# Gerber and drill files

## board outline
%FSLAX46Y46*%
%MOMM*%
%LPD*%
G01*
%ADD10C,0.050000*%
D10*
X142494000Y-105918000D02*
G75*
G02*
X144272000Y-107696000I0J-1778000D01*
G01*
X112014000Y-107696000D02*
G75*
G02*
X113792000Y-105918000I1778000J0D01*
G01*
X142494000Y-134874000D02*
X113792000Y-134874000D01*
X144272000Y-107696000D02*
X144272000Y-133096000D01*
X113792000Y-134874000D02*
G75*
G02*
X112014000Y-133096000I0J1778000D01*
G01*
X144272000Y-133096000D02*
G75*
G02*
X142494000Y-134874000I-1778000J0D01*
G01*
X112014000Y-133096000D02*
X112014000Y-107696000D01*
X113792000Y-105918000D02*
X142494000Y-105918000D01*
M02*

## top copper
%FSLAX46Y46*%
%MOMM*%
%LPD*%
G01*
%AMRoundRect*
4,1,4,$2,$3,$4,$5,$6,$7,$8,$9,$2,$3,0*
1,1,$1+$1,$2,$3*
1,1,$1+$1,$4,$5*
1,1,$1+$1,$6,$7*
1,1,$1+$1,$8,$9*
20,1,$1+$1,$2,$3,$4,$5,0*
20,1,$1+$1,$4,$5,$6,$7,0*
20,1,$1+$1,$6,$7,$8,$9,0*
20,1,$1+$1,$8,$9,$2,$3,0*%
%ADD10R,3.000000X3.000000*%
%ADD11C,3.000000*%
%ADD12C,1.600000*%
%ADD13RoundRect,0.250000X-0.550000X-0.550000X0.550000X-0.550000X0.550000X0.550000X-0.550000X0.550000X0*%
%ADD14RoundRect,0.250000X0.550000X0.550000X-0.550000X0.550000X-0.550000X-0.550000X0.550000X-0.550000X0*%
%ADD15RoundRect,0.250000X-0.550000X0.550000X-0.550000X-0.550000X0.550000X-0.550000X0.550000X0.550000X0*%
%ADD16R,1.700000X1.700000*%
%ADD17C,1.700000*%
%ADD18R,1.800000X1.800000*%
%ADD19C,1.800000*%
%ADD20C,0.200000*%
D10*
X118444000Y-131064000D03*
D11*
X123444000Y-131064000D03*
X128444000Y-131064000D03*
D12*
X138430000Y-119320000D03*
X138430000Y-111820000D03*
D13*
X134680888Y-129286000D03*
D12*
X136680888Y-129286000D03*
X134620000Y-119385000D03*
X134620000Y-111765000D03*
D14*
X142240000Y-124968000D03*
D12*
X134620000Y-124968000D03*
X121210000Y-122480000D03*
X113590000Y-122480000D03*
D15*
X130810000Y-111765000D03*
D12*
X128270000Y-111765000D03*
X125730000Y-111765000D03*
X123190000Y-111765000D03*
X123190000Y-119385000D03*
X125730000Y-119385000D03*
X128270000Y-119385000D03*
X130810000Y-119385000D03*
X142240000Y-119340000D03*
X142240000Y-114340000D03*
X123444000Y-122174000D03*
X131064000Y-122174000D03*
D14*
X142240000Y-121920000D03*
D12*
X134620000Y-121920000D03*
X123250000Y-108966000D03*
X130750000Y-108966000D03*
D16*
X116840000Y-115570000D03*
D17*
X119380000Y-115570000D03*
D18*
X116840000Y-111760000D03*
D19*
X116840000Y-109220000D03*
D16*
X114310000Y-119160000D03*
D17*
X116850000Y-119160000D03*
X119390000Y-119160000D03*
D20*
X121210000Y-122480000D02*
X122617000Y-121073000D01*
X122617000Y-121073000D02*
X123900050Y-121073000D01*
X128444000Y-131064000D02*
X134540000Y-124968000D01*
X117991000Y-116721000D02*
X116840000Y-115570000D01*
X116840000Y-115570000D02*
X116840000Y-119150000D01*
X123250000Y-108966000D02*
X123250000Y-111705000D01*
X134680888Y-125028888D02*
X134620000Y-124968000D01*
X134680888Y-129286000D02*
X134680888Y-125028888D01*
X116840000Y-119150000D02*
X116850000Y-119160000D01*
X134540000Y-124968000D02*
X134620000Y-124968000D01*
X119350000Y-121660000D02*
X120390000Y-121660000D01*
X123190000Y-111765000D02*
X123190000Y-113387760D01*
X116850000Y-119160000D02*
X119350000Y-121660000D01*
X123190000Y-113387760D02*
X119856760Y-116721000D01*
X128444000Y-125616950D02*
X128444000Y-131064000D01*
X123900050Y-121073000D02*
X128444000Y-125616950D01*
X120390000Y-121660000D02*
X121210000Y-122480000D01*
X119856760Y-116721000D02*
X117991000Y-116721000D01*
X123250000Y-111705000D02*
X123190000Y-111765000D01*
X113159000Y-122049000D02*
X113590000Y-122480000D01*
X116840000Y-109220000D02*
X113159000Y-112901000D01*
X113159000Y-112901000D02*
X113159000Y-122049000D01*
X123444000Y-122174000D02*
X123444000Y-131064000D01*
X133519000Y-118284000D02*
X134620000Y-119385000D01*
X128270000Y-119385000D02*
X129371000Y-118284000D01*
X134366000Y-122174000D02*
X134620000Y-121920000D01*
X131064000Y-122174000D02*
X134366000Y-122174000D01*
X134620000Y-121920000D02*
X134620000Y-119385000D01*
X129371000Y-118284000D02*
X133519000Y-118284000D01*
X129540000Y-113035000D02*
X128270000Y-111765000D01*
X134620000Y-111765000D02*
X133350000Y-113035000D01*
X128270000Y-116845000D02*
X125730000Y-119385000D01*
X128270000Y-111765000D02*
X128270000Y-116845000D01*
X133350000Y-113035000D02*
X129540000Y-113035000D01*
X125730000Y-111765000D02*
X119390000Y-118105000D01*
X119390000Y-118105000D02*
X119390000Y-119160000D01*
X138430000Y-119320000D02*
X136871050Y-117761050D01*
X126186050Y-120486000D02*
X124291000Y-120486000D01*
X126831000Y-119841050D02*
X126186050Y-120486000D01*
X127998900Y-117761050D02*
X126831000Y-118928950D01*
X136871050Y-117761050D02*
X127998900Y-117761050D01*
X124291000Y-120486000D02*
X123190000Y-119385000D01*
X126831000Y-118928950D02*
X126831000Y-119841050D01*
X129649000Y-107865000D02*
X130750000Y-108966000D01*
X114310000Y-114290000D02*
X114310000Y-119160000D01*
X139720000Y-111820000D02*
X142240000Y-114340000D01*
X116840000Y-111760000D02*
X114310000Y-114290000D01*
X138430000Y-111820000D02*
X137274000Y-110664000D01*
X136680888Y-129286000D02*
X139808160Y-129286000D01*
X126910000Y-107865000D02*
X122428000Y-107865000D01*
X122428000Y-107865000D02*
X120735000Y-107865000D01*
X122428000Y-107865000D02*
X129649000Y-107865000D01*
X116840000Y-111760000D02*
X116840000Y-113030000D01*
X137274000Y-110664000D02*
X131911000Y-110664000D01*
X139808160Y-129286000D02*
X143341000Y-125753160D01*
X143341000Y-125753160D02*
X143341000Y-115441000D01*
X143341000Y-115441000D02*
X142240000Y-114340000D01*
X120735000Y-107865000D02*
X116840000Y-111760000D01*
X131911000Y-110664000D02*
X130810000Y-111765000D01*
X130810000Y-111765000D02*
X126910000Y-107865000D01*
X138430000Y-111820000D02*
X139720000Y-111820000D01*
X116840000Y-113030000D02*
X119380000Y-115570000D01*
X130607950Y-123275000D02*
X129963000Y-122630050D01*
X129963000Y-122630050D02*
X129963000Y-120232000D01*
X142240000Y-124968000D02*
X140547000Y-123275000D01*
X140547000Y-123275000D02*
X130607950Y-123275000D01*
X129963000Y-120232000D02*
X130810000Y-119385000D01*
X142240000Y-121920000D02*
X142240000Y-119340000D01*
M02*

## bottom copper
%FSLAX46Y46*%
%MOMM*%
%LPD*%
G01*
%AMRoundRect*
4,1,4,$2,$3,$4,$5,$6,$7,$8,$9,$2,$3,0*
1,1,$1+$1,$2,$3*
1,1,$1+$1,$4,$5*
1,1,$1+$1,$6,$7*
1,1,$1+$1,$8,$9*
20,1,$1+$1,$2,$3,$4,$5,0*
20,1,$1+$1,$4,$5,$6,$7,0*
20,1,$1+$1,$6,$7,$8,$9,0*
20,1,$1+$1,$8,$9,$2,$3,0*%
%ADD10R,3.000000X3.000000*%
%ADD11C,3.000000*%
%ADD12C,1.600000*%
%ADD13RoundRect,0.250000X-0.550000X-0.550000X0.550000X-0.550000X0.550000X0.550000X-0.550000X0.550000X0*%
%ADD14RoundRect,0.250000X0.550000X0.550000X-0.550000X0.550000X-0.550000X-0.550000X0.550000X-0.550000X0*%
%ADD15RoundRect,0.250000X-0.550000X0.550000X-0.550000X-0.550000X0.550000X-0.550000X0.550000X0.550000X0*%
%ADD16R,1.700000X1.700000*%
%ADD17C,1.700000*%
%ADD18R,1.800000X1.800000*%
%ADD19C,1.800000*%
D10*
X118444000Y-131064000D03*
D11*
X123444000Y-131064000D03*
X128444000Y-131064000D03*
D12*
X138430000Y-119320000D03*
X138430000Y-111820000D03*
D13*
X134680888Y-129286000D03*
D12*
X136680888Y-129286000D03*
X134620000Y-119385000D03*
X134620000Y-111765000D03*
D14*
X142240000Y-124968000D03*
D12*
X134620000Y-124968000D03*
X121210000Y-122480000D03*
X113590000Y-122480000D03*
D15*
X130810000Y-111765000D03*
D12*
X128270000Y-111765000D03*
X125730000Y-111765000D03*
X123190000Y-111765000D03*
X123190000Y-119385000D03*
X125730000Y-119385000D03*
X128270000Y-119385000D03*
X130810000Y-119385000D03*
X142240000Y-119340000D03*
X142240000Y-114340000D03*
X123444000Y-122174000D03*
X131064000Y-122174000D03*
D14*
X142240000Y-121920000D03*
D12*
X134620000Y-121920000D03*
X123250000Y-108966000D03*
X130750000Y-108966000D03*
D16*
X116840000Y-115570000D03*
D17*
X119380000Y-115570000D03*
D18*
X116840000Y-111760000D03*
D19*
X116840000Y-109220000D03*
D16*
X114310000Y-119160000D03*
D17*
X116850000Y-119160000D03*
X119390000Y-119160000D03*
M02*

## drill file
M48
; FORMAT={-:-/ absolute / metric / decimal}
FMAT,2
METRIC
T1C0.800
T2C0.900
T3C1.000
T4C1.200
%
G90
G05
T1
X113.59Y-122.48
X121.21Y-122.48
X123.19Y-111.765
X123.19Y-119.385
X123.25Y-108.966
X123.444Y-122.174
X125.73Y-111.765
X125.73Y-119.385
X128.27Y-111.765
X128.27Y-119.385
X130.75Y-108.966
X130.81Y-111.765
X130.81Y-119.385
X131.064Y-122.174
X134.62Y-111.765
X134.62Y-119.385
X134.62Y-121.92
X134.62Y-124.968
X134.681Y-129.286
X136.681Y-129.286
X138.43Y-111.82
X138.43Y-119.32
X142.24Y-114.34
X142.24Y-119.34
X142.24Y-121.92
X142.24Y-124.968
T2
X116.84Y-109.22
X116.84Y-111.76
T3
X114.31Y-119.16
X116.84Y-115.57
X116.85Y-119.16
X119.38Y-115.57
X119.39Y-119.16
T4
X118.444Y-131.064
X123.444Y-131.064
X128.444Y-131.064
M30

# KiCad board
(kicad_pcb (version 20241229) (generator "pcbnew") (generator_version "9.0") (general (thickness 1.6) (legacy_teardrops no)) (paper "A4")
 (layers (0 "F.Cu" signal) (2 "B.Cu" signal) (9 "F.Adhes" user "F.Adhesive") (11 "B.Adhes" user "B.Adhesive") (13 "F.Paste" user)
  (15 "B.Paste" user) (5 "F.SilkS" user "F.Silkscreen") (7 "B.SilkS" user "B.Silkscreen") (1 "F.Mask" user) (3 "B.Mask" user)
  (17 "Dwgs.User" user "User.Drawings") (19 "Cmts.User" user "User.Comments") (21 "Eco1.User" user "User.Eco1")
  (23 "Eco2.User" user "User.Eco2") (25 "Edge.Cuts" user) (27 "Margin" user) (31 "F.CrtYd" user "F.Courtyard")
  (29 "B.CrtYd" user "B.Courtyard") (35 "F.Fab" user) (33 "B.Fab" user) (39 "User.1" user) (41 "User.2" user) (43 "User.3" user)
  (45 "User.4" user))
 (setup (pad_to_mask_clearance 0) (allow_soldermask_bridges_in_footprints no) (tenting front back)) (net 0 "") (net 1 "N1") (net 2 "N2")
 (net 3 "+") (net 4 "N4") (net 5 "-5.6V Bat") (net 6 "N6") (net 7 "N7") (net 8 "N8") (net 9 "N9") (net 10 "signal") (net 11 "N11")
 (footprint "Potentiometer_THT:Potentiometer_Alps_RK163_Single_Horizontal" (layer "F.Cu") (at 118.444 131.064 90)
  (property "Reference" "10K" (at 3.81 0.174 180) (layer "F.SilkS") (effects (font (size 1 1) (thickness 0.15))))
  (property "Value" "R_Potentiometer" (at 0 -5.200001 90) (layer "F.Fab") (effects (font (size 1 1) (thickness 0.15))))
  (pad "1" thru_hole rect (at 0 0 270) (size 3 3) (drill 1.2) (layers "*.Cu" "*.Mask") (remove_unused_layers no) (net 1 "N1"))
  (pad "2" thru_hole circle (at 0 5 270) (size 3 3) (drill 1.2) (layers "*.Cu" "*.Mask") (remove_unused_layers no) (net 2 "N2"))
  (pad "3" thru_hole circle (at 0 10 270) (size 3 3) (drill 1.2) (layers "*.Cu" "*.Mask") (remove_unused_layers no) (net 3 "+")))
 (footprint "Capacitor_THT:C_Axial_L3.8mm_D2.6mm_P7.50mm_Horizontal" (layer "F.Cu") (at 138.43 119.32 90)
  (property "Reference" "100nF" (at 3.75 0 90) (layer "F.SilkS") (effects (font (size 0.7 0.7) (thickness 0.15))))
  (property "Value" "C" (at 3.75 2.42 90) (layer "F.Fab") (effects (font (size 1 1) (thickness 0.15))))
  (pad "1" thru_hole circle (at 0 0 90) (size 1.6 1.6) (drill 0.8) (layers "*.Cu" "*.Mask") (remove_unused_layers no) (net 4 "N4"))
  (pad "2" thru_hole circle (at 7.5 0 90) (size 1.6 1.6) (drill 0.8) (layers "*.Cu" "*.Mask") (remove_unused_layers no) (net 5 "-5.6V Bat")))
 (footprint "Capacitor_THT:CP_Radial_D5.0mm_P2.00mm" (layer "F.Cu") (at 134.680888 129.286)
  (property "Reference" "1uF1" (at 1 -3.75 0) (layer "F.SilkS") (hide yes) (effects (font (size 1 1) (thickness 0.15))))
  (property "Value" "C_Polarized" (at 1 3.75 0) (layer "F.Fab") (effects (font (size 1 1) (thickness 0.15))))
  (pad "1" thru_hole roundrect (at 0 0) (size 1.6 1.6) (drill 0.8) (layers "*.Cu" "*.Mask") (remove_unused_layers no)
   (roundrect_rratio 0.15625) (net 3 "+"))
  (pad "2" thru_hole circle (at 2 0) (size 1.6 1.6) (drill 0.8) (layers "*.Cu" "*.Mask") (remove_unused_layers no) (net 5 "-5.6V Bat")))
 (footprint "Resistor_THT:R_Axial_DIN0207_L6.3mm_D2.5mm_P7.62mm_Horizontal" (layer "F.Cu") (at 134.62 119.385 90)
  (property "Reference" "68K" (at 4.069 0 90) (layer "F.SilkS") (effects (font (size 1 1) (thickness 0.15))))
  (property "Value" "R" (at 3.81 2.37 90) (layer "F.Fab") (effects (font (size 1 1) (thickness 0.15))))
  (pad "1" thru_hole circle (at 0 0 90) (size 1.6 1.6) (drill 0.8) (layers "*.Cu" "*.Mask") (remove_unused_layers no) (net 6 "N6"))
  (pad "2" thru_hole circle (at 7.62 0 90) (size 1.6 1.6) (drill 0.8) (layers "*.Cu" "*.Mask") (remove_unused_layers no) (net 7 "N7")))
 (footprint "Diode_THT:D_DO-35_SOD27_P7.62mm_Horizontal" (layer "F.Cu") (at 142.24 124.968 180)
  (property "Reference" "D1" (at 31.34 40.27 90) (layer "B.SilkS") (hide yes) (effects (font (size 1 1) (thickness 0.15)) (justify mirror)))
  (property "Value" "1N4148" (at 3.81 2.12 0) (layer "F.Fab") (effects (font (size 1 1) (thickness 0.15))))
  (pad "1" thru_hole roundrect (at 0 0 180) (size 1.6 1.6) (drill 0.8) (layers "*.Cu" "*.Mask") (remove_unused_layers no)
   (roundrect_rratio 0.15625) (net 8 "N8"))
  (pad "2" thru_hole circle (at 7.62 0 180) (size 1.6 1.6) (drill 0.8) (layers "*.Cu" "*.Mask") (remove_unused_layers no) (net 3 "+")))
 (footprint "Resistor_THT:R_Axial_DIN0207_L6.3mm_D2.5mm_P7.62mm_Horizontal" (layer "F.Cu") (at 121.21 122.48 180)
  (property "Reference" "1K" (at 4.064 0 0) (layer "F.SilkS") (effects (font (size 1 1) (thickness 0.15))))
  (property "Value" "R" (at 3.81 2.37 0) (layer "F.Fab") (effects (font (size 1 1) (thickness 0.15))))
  (pad "1" thru_hole circle (at 0 0 180) (size 1.6 1.6) (drill 0.8) (layers "*.Cu" "*.Mask") (remove_unused_layers no) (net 3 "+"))
  (pad "2" thru_hole circle (at 7.62 0 180) (size 1.6 1.6) (drill 0.8) (layers "*.Cu" "*.Mask") (remove_unused_layers no) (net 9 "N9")))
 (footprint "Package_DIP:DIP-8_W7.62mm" (layer "F.Cu") (at 130.81 111.765 -90)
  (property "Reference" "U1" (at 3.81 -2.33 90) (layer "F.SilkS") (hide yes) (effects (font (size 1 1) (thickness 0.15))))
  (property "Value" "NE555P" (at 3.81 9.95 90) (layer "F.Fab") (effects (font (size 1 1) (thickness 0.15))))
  (pad "1" thru_hole roundrect (at 0 0 270) (size 1.6 1.6) (drill 0.8) (layers "*.Cu" "*.Mask") (remove_unused_layers no)
   (roundrect_rratio 0.15625) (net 5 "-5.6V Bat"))
  (pad "2" thru_hole circle (at 0 2.54 270) (size 1.6 1.6) (drill 0.8) (layers "*.Cu" "*.Mask") (remove_unused_layers no) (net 7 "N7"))
  (pad "3" thru_hole circle (at 0 5.08 270) (size 1.6 1.6) (drill 0.8) (layers "*.Cu" "*.Mask") (remove_unused_layers no) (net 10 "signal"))
  (pad "4" thru_hole circle (at 0 7.62 270) (size 1.6 1.6) (drill 0.8) (layers "*.Cu" "*.Mask") (remove_unused_layers no) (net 3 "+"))
  (pad "5" thru_hole circle (at 7.62 7.62 270) (size 1.6 1.6) (drill 0.8) (layers "*.Cu" "*.Mask") (remove_unused_layers no) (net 4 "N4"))
  (pad "6" thru_hole circle (at 7.62 5.08 270) (size 1.6 1.6) (drill 0.8) (layers "*.Cu" "*.Mask") (remove_unused_layers no) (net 7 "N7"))
  (pad "7" thru_hole circle (at 7.62 2.54 270) (size 1.6 1.6) (drill 0.8) (layers "*.Cu" "*.Mask") (remove_unused_layers no) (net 6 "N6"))
  (pad "8" thru_hole circle (at 7.62 0 270) (size 1.6 1.6) (drill 0.8) (layers "*.Cu" "*.Mask") (remove_unused_layers no) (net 8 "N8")))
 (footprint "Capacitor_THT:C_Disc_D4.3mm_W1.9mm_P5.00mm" (layer "F.Cu") (at 142.24 119.34 90)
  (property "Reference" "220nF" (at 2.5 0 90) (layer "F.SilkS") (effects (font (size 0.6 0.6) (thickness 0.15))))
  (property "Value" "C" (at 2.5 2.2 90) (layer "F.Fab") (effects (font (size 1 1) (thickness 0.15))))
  (pad "1" thru_hole circle (at 0 0 90) (size 1.6 1.6) (drill 0.8) (layers "*.Cu" "*.Mask") (remove_unused_layers no) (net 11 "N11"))
  (pad "2" thru_hole circle (at 5 0 90) (size 1.6 1.6) (drill 0.8) (layers "*.Cu" "*.Mask") (remove_unused_layers no) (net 5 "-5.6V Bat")))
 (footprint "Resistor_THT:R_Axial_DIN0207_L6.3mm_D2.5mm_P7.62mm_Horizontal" (layer "F.Cu") (at 123.444 122.174)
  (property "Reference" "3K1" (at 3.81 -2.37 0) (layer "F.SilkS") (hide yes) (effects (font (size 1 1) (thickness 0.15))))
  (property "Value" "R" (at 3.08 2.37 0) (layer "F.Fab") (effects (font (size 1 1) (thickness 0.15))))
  (pad "1" thru_hole circle (at 0 0) (size 1.6 1.6) (drill 0.8) (layers "*.Cu" "*.Mask") (remove_unused_layers no) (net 2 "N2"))
  (pad "2" thru_hole circle (at 7.62 0) (size 1.6 1.6) (drill 0.8) (layers "*.Cu" "*.Mask") (remove_unused_layers no) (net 6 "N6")))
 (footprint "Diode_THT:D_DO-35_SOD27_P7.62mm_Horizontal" (layer "F.Cu") (at 142.24 121.92 180)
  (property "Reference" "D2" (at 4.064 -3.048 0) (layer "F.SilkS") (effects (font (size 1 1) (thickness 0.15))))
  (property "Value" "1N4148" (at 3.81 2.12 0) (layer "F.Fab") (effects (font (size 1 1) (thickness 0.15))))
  (pad "1" thru_hole roundrect (at 0 0 180) (size 1.6 1.6) (drill 0.8) (layers "*.Cu" "*.Mask") (remove_unused_layers no)
   (roundrect_rratio 0.15625) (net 11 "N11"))
  (pad "2" thru_hole circle (at 7.62 0 180) (size 1.6 1.6) (drill 0.8) (layers "*.Cu" "*.Mask") (remove_unused_layers no) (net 6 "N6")))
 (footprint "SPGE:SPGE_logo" (layer "F.Cu") (at 141 108.8)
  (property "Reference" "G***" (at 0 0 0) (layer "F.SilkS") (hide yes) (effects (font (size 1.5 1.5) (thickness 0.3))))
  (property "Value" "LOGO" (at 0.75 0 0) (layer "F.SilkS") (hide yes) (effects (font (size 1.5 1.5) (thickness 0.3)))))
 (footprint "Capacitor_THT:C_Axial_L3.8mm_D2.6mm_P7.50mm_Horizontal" (layer "F.Cu") (at 123.25 108.966)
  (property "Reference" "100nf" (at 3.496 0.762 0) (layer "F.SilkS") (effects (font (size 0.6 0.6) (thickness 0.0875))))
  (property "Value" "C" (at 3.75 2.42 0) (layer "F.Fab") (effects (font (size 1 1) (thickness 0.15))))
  (pad "1" thru_hole circle (at 0 0) (size 1.6 1.6) (drill 0.8) (layers "*.Cu" "*.Mask") (remove_unused_layers no) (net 3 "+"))
  (pad "2" thru_hole circle (at 7.5 0) (size 1.6 1.6) (drill 0.8) (layers "*.Cu" "*.Mask") (remove_unused_layers no) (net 5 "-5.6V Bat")))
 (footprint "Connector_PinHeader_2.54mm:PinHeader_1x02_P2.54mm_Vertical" (layer "F.Cu") (at 116.84 115.57 90)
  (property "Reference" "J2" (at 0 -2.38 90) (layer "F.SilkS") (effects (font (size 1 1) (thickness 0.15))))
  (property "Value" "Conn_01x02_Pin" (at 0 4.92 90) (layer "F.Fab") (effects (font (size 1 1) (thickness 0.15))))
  (pad "1" thru_hole rect (at 0 0 90) (size 1.7 1.7) (drill 1) (layers "*.Cu" "*.Mask") (remove_unused_layers no) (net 3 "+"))
  (pad "2" thru_hole circle (at 0 2.54 90) (size 1.7 1.7) (drill 1) (layers "*.Cu" "*.Mask") (remove_unused_layers no) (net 5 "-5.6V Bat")))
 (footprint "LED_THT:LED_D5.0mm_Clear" (layer "F.Cu") (at 116.84 111.76 90)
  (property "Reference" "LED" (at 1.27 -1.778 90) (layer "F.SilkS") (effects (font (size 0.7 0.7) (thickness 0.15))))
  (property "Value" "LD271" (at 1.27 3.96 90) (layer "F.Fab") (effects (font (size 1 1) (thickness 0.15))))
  (pad "1" thru_hole rect (at 0 0 90) (size 1.8 1.8) (drill 0.9) (layers "*.Cu" "*.Mask") (remove_unused_layers no) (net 5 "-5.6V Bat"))
  (pad "2" thru_hole circle (at 2.54 0 90) (size 1.8 1.8) (drill 0.9) (layers "*.Cu" "*.Mask") (remove_unused_layers no) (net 9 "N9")))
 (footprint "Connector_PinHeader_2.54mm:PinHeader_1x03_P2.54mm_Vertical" (layer "F.Cu") (at 114.31 119.16 90)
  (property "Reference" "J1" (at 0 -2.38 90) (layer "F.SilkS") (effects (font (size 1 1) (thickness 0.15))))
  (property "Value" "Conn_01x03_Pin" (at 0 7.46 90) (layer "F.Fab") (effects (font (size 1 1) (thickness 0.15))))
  (pad "1" thru_hole rect (at 0 0 90) (size 1.7 1.7) (drill 1) (layers "*.Cu" "*.Mask") (remove_unused_layers no) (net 5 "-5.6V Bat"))
  (pad "2" thru_hole circle (at 0 2.54 90) (size 1.7 1.7) (drill 1) (layers "*.Cu" "*.Mask") (remove_unused_layers no) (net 3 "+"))
  (pad "3" thru_hole circle (at 0 5.08 90) (size 1.7 1.7) (drill 1) (layers "*.Cu" "*.Mask") (remove_unused_layers no) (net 10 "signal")))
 (gr_arc (start 142.494 105.918) (mid 143.751236 106.438764) (end 144.272 107.696) (stroke (width 0.05) (type default)) (layer "Edge.Cuts"))
 (gr_arc (start 112.014 107.696) (mid 112.534764 106.438764) (end 113.792 105.918) (stroke (width 0.05) (type default)) (layer "Edge.Cuts"))
 (gr_line (start 142.494 134.874) (end 113.792 134.874) (stroke (width 0.05) (type default)) (layer "Edge.Cuts"))
 (gr_line (start 144.272 107.696) (end 144.272 133.096) (stroke (width 0.05) (type default)) (layer "Edge.Cuts"))
 (gr_arc (start 113.792 134.874) (mid 112.534764 134.353236) (end 112.014 133.096) (stroke (width 0.05) (type default)) (layer "Edge.Cuts"))
 (gr_arc (start 144.272 133.096) (mid 143.751236 134.353236) (end 142.494 134.874) (stroke (width 0.05) (type default)) (layer "Edge.Cuts"))
 (gr_line (start 112.014 133.096) (end 112.014 107.696) (stroke (width 0.05) (type default)) (layer "Edge.Cuts"))
 (gr_line (start 113.792 105.918) (end 142.494 105.918) (stroke (width 0.05) (type default)) (layer "Edge.Cuts"))
 (segment (start 121.21 122.48) (end 122.617 121.073) (width 0.2) (layer "F.Cu") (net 3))
 (segment (start 122.617 121.073) (end 123.90005 121.073) (width 0.2) (layer "F.Cu") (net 3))
 (segment (start 128.444 131.064) (end 134.54 124.968) (width 0.2) (layer "F.Cu") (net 3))
 (segment (start 117.991 116.721) (end 116.84 115.57) (width 0.2) (layer "F.Cu") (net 3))
 (segment (start 116.84 115.57) (end 116.84 119.15) (width 0.2) (layer "F.Cu") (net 3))
 (segment (start 123.25 108.966) (end 123.25 111.705) (width 0.2) (layer "F.Cu") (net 3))
 (segment (start 134.680888 125.028888) (end 134.62 124.968) (width 0.2) (layer "F.Cu") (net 3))
 (segment (start 134.680888 129.286) (end 134.680888 125.028888) (width 0.2) (layer "F.Cu") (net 3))
 (segment (start 116.84 119.15) (end 116.85 119.16) (width 0.2) (layer "F.Cu") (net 3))
 (segment (start 134.54 124.968) (end 134.62 124.968) (width 0.2) (layer "F.Cu") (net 3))
 (segment (start 119.35 121.66) (end 120.39 121.66) (width 0.2) (layer "F.Cu") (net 3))
 (segment (start 123.19 111.765) (end 123.19 113.38776) (width 0.2) (layer "F.Cu") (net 3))
 (segment (start 116.85 119.16) (end 119.35 121.66) (width 0.2) (layer "F.Cu") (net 3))
 (segment (start 123.19 113.38776) (end 119.85676 116.721) (width 0.2) (layer "F.Cu") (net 3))
 (segment (start 128.444 125.61695) (end 128.444 131.064) (width 0.2) (layer "F.Cu") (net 3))
 (segment (start 123.90005 121.073) (end 128.444 125.61695) (width 0.2) (layer "F.Cu") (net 3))
 (segment (start 120.39 121.66) (end 121.21 122.48) (width 0.2) (layer "F.Cu") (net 3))
 (segment (start 119.85676 116.721) (end 117.991 116.721) (width 0.2) (layer "F.Cu") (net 3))
 (segment (start 123.25 111.705) (end 123.19 111.765) (width 0.2) (layer "F.Cu") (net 3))
 (segment (start 113.159 122.049) (end 113.59 122.48) (width 0.2) (layer "F.Cu") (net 9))
 (segment (start 116.84 109.22) (end 113.159 112.901) (width 0.2) (layer "F.Cu") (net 9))
 (segment (start 113.159 112.901) (end 113.159 122.049) (width 0.2) (layer "F.Cu") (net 9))
 (segment (start 123.444 122.174) (end 123.444 131.064) (width 0.2) (layer "F.Cu") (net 2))
 (segment (start 133.519 118.284) (end 134.62 119.385) (width 0.2) (layer "F.Cu") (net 6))
 (segment (start 128.27 119.385) (end 129.371 118.284) (width 0.2) (layer "F.Cu") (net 6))
 (segment (start 134.366 122.174) (end 134.62 121.92) (width 0.2) (layer "F.Cu") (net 6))
 (segment (start 131.064 122.174) (end 134.366 122.174) (width 0.2) (layer "F.Cu") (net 6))
 (segment (start 134.62 121.92) (end 134.62 119.385) (width 0.2) (layer "F.Cu") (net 6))
 (segment (start 129.371 118.284) (end 133.519 118.284) (width 0.2) (layer "F.Cu") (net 6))
 (segment (start 129.54 113.035) (end 128.27 111.765) (width 0.2) (layer "F.Cu") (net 7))
 (segment (start 134.62 111.765) (end 133.35 113.035) (width 0.2) (layer "F.Cu") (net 7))
 (segment (start 128.27 116.845) (end 125.73 119.385) (width 0.2) (layer "F.Cu") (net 7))
 (segment (start 128.27 111.765) (end 128.27 116.845) (width 0.2) (layer "F.Cu") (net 7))
 (segment (start 133.35 113.035) (end 129.54 113.035) (width 0.2) (layer "F.Cu") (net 7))
 (segment (start 125.73 111.765) (end 119.39 118.105) (width 0.2) (layer "F.Cu") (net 10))
 (segment (start 119.39 118.105) (end 119.39 119.16) (width 0.2) (layer "F.Cu") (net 10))
 (segment (start 138.43 119.32) (end 136.87105 117.76105) (width 0.2) (layer "F.Cu") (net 4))
 (segment (start 126.18605 120.486) (end 124.291 120.486) (width 0.2) (layer "F.Cu") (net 4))
 (segment (start 126.831 119.84105) (end 126.18605 120.486) (width 0.2) (layer "F.Cu") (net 4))
 (segment (start 127.9989 117.76105) (end 126.831 118.92895) (width 0.2) (layer "F.Cu") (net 4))
 (segment (start 136.87105 117.76105) (end 127.9989 117.76105) (width 0.2) (layer "F.Cu") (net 4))
 (segment (start 124.291 120.486) (end 123.19 119.385) (width 0.2) (layer "F.Cu") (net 4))
 (segment (start 126.831 118.92895) (end 126.831 119.84105) (width 0.2) (layer "F.Cu") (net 4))
 (segment (start 129.649 107.865) (end 130.75 108.966) (width 0.2) (layer "F.Cu") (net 5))
 (segment (start 114.31 114.29) (end 114.31 119.16) (width 0.2) (layer "F.Cu") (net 5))
 (segment (start 139.72 111.82) (end 142.24 114.34) (width 0.2) (layer "F.Cu") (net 5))
 (segment (start 116.84 111.76) (end 114.31 114.29) (width 0.2) (layer "F.Cu") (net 5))
 (segment (start 138.43 111.82) (end 137.274 110.664) (width 0.2) (layer "F.Cu") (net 5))
 (segment (start 136.680888 129.286) (end 139.80816 129.286) (width 0.2) (layer "F.Cu") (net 5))
 (segment (start 126.91 107.865) (end 122.428 107.865) (width 0.2) (layer "F.Cu") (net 5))
 (segment (start 122.428 107.865) (end 120.735 107.865) (width 0.2) (layer "F.Cu") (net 5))
 (segment (start 122.428 107.865) (end 129.649 107.865) (width 0.2) (layer "F.Cu") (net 5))
 (segment (start 116.84 111.76) (end 116.84 113.03) (width 0.2) (layer "F.Cu") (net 5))
 (segment (start 137.274 110.664) (end 131.911 110.664) (width 0.2) (layer "F.Cu") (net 5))
 (segment (start 139.80816 129.286) (end 143.341 125.75316) (width 0.2) (layer "F.Cu") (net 5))
 (segment (start 143.341 125.75316) (end 143.341 115.441) (width 0.2) (layer "F.Cu") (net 5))
 (segment (start 143.341 115.441) (end 142.24 114.34) (width 0.2) (layer "F.Cu") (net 5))
 (segment (start 120.735 107.865) (end 116.84 111.76) (width 0.2) (layer "F.Cu") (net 5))
 (segment (start 131.911 110.664) (end 130.81 111.765) (width 0.2) (layer "F.Cu") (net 5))
 (segment (start 130.81 111.765) (end 126.91 107.865) (width 0.2) (layer "F.Cu") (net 5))
 (segment (start 138.43 111.82) (end 139.72 111.82) (width 0.2) (layer "F.Cu") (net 5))
 (segment (start 116.84 113.03) (end 119.38 115.57) (width 0.2) (layer "F.Cu") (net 5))
 (segment (start 130.60795 123.275) (end 129.963 122.63005) (width 0.2) (layer "F.Cu") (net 8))
 (segment (start 129.963 122.63005) (end 129.963 120.232) (width 0.2) (layer "F.Cu") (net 8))
 (segment (start 142.24 124.968) (end 140.547 123.275) (width 0.2) (layer "F.Cu") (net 8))
 (segment (start 140.547 123.275) (end 130.60795 123.275) (width 0.2) (layer "F.Cu") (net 8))
 (segment (start 129.963 120.232) (end 130.81 119.385) (width 0.2) (layer "F.Cu") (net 8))
 (segment (start 142.24 121.92) (end 142.24 119.34) (width 0.2) (layer "F.Cu") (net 11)))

